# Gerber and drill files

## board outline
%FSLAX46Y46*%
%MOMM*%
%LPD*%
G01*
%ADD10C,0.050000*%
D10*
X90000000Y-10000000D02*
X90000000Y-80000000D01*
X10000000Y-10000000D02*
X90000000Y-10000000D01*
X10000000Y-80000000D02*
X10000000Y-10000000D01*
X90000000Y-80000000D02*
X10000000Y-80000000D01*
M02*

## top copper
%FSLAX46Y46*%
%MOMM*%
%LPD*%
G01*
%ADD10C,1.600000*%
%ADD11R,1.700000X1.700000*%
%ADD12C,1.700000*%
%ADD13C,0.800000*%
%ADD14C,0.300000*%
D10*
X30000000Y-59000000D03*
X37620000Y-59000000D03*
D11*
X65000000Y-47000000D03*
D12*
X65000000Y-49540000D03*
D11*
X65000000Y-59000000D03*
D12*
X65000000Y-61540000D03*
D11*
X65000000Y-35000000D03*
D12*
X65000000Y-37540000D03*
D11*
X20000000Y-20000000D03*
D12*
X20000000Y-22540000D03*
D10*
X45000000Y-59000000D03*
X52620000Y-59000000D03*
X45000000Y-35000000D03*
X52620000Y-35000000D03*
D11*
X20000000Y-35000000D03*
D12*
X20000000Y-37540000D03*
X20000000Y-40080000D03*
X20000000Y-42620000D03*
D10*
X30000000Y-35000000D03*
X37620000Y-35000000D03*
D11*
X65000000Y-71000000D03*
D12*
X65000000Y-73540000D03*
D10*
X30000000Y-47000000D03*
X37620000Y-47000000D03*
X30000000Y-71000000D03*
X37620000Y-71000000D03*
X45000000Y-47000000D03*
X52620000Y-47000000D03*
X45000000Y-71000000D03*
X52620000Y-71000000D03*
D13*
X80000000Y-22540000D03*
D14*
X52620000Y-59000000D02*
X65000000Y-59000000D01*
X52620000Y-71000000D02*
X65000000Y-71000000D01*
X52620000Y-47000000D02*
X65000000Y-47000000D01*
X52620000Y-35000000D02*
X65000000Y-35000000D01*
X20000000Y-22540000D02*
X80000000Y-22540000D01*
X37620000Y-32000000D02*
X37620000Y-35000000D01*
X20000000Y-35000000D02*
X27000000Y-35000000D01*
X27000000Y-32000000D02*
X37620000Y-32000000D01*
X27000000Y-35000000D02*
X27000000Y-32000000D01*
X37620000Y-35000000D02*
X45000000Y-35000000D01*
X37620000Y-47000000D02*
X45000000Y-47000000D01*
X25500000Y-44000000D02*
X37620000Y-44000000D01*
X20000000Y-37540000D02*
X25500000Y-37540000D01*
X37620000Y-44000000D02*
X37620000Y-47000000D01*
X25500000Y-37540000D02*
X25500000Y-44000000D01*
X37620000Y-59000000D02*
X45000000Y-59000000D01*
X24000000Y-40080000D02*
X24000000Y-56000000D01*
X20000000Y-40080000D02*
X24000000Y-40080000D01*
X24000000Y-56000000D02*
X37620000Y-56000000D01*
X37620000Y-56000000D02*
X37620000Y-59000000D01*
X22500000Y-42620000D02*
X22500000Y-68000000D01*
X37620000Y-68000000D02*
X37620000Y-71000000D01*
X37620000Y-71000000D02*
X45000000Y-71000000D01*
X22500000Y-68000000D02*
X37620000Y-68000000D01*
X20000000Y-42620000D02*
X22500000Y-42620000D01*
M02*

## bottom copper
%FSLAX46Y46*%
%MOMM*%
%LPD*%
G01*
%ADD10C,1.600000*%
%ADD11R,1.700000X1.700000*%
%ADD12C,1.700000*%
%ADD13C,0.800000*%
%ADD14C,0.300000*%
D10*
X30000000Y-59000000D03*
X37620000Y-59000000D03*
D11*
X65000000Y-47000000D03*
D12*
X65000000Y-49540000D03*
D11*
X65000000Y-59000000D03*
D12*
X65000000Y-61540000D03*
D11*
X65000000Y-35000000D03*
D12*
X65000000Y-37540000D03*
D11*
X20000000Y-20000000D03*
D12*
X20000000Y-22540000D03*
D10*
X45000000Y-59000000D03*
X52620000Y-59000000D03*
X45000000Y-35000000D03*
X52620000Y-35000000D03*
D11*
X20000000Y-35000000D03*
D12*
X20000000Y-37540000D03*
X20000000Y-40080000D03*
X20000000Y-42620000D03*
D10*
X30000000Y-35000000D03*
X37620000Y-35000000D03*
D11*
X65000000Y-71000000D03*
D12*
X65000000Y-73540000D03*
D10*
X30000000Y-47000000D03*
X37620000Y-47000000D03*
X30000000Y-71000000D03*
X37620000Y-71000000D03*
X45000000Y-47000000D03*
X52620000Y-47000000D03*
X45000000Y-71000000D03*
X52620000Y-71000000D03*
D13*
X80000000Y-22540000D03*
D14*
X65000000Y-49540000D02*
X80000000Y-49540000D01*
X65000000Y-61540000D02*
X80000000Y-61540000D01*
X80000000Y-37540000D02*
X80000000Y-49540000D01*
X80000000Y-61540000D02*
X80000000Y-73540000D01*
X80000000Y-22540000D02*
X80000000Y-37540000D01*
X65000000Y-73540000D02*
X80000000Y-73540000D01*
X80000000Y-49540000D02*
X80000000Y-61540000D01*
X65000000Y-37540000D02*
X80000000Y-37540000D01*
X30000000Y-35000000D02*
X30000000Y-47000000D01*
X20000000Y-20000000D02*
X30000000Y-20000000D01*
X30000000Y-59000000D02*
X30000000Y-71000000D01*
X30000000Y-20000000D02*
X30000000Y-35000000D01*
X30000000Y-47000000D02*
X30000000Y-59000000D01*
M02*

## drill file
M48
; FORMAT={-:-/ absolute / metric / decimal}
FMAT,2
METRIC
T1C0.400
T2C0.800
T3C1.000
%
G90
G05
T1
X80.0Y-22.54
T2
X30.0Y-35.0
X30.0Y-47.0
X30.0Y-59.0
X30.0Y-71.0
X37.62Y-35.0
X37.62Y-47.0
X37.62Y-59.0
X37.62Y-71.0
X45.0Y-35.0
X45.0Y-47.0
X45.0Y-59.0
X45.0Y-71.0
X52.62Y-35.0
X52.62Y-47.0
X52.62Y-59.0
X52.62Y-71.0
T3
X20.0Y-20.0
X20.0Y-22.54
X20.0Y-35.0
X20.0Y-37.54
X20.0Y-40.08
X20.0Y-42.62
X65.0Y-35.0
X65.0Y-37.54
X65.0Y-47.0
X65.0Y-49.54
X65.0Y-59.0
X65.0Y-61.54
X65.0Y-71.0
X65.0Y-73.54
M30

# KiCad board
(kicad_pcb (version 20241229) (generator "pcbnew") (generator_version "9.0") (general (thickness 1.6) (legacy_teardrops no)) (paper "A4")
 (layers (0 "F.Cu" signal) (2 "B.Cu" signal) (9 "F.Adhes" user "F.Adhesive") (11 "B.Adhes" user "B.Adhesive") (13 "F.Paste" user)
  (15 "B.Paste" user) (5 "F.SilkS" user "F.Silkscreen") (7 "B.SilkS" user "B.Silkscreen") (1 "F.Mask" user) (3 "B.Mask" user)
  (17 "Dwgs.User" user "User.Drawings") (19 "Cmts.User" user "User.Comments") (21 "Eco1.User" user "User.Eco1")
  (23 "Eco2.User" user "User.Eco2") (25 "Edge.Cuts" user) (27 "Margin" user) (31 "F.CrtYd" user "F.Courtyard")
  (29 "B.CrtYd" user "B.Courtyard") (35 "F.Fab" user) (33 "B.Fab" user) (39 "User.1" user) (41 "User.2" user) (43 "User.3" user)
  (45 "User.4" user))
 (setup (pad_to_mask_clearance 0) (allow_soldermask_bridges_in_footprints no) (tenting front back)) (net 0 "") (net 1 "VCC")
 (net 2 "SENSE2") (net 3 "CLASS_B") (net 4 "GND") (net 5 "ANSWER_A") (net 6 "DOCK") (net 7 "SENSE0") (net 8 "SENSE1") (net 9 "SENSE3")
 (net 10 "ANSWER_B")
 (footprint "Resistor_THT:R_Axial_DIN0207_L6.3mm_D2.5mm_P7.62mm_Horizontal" (layer "F.Cu") (at 30 59)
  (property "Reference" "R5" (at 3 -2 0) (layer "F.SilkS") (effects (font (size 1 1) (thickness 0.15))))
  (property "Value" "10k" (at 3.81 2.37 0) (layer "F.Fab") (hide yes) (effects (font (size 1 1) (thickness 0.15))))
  (pad "1" thru_hole circle (at 0 0) (size 1.6 1.6) (drill 0.8) (layers "*.Cu" "*.Mask") (remove_unused_layers no) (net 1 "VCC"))
  (pad "2" thru_hole circle (at 7.62 0) (size 1.6 1.6) (drill 0.8) (layers "*.Cu" "*.Mask") (remove_unused_layers no) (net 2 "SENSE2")))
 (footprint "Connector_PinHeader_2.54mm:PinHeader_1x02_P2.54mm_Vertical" (layer "F.Cu") (at 65 47)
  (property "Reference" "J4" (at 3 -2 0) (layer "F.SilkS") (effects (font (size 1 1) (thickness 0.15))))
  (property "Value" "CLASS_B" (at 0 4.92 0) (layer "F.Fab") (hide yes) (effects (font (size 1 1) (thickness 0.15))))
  (pad "1" thru_hole rect (at 0 0) (size 1.7 1.7) (drill 1) (layers "*.Cu" "*.Mask") (remove_unused_layers no) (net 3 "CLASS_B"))
  (pad "2" thru_hole circle (at 0 2.54) (size 1.7 1.7) (drill 1) (layers "*.Cu" "*.Mask") (remove_unused_layers no) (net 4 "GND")))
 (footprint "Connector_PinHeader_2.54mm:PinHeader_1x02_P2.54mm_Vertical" (layer "F.Cu") (at 65 59)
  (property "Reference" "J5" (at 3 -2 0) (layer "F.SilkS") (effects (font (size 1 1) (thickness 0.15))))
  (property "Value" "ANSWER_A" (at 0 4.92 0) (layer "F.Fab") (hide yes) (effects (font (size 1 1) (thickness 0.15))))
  (pad "1" thru_hole rect (at 0 0) (size 1.7 1.7) (drill 1) (layers "*.Cu" "*.Mask") (remove_unused_layers no) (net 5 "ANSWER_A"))
  (pad "2" thru_hole circle (at 0 2.54) (size 1.7 1.7) (drill 1) (layers "*.Cu" "*.Mask") (remove_unused_layers no) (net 4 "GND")))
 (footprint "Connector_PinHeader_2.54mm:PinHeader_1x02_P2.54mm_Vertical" (layer "F.Cu") (at 65 35)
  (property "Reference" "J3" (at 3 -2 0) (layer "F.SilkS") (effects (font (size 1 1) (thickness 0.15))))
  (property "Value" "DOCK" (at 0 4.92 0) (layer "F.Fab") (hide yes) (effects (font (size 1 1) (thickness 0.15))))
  (pad "1" thru_hole rect (at 0 0) (size 1.7 1.7) (drill 1) (layers "*.Cu" "*.Mask") (remove_unused_layers no) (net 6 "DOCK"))
  (pad "2" thru_hole circle (at 0 2.54) (size 1.7 1.7) (drill 1) (layers "*.Cu" "*.Mask") (remove_unused_layers no) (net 4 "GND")))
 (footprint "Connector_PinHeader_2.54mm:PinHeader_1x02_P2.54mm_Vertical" (layer "F.Cu") (at 20 20)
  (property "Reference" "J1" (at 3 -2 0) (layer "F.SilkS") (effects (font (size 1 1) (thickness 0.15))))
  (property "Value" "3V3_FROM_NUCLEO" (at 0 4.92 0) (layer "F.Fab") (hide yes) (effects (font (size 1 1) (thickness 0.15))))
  (pad "1" thru_hole rect (at 0 0) (size 1.7 1.7) (drill 1) (layers "*.Cu" "*.Mask") (remove_unused_layers no) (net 1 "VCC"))
  (pad "2" thru_hole circle (at 0 2.54) (size 1.7 1.7) (drill 1) (layers "*.Cu" "*.Mask") (remove_unused_layers no) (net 4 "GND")))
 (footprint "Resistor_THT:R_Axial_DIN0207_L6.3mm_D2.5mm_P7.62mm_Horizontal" (layer "F.Cu") (at 45 59)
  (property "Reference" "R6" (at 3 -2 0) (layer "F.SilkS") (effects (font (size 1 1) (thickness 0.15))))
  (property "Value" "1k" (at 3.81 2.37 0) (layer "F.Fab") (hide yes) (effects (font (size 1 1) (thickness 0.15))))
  (pad "1" thru_hole circle (at 0 0) (size 1.6 1.6) (drill 0.8) (layers "*.Cu" "*.Mask") (remove_unused_layers no) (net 2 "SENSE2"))
  (pad "2" thru_hole circle (at 7.62 0) (size 1.6 1.6) (drill 0.8) (layers "*.Cu" "*.Mask") (remove_unused_layers no) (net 5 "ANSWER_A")))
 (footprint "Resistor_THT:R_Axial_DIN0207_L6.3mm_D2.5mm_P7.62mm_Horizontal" (layer "F.Cu") (at 45 35)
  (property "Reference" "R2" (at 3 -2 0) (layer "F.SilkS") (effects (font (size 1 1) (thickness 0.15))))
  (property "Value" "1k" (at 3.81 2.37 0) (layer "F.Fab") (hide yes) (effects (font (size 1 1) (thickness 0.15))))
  (pad "1" thru_hole circle (at 0 0) (size 1.6 1.6) (drill 0.8) (layers "*.Cu" "*.Mask") (remove_unused_layers no) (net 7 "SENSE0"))
  (pad "2" thru_hole circle (at 7.62 0) (size 1.6 1.6) (drill 0.8) (layers "*.Cu" "*.Mask") (remove_unused_layers no) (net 6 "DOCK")))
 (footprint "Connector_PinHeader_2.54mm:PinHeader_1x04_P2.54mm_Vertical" (layer "F.Cu") (at 20 35)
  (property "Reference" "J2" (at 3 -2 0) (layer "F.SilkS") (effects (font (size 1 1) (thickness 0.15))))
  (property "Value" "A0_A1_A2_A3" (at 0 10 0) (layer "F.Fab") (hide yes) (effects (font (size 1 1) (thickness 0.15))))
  (pad "1" thru_hole rect (at 0 0) (size 1.7 1.7) (drill 1) (layers "*.Cu" "*.Mask") (remove_unused_layers no) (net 7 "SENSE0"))
  (pad "2" thru_hole circle (at 0 2.54) (size 1.7 1.7) (drill 1) (layers "*.Cu" "*.Mask") (remove_unused_layers no) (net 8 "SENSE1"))
  (pad "3" thru_hole circle (at 0 5.08) (size 1.7 1.7) (drill 1) (layers "*.Cu" "*.Mask") (remove_unused_layers no) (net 2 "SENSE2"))
  (pad "4" thru_hole circle (at 0 7.62) (size 1.7 1.7) (drill 1) (layers "*.Cu" "*.Mask") (remove_unused_layers no) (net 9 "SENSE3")))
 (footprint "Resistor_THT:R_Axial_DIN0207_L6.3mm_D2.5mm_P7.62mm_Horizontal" (layer "F.Cu") (at 30 35)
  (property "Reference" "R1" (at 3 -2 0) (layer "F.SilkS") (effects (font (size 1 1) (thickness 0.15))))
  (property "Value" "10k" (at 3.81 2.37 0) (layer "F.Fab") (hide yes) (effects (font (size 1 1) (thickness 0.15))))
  (pad "1" thru_hole circle (at 0 0) (size 1.6 1.6) (drill 0.8) (layers "*.Cu" "*.Mask") (remove_unused_layers no) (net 1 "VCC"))
  (pad "2" thru_hole circle (at 7.62 0) (size 1.6 1.6) (drill 0.8) (layers "*.Cu" "*.Mask") (remove_unused_layers no) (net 7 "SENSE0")))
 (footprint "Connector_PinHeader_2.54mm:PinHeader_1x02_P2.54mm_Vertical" (layer "F.Cu") (at 65 71)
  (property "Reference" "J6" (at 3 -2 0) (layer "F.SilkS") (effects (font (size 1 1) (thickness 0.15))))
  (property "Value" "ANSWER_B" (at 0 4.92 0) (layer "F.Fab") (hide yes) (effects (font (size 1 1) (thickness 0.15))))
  (pad "1" thru_hole rect (at 0 0) (size 1.7 1.7) (drill 1) (layers "*.Cu" "*.Mask") (remove_unused_layers no) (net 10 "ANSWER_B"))
  (pad "2" thru_hole circle (at 0 2.54) (size 1.7 1.7) (drill 1) (layers "*.Cu" "*.Mask") (remove_unused_layers no) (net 4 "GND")))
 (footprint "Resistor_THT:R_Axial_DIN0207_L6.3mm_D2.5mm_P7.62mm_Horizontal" (layer "F.Cu") (at 30 47)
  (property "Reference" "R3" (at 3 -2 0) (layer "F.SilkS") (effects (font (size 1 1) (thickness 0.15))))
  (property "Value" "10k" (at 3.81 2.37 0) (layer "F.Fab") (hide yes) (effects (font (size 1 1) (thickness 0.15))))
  (pad "1" thru_hole circle (at 0 0) (size 1.6 1.6) (drill 0.8) (layers "*.Cu" "*.Mask") (remove_unused_layers no) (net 1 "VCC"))
  (pad "2" thru_hole circle (at 7.62 0) (size 1.6 1.6) (drill 0.8) (layers "*.Cu" "*.Mask") (remove_unused_layers no) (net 8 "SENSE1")))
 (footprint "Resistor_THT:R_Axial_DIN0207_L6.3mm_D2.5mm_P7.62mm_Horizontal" (layer "F.Cu") (at 30 71)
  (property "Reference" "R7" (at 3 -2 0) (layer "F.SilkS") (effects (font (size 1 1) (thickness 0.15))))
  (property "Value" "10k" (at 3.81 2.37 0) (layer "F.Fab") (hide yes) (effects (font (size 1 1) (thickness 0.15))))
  (pad "1" thru_hole circle (at 0 0) (size 1.6 1.6) (drill 0.8) (layers "*.Cu" "*.Mask") (remove_unused_layers no) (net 1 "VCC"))
  (pad "2" thru_hole circle (at 7.62 0) (size 1.6 1.6) (drill 0.8) (layers "*.Cu" "*.Mask") (remove_unused_layers no) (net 9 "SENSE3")))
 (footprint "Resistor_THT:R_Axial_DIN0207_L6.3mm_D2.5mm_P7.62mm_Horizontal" (layer "F.Cu") (at 45 47)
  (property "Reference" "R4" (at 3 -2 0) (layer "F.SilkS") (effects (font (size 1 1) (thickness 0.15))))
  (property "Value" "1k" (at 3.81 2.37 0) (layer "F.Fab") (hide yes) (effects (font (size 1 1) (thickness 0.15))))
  (pad "1" thru_hole circle (at 0 0) (size 1.6 1.6) (drill 0.8) (layers "*.Cu" "*.Mask") (remove_unused_layers no) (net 8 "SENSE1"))
  (pad "2" thru_hole circle (at 7.62 0) (size 1.6 1.6) (drill 0.8) (layers "*.Cu" "*.Mask") (remove_unused_layers no) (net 3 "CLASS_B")))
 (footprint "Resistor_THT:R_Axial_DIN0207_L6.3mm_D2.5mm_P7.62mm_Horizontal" (layer "F.Cu") (at 45 71)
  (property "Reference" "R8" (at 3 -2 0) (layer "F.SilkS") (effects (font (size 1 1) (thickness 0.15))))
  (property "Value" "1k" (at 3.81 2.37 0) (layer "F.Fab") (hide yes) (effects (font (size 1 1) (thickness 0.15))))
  (pad "1" thru_hole circle (at 0 0) (size 1.6 1.6) (drill 0.8) (layers "*.Cu" "*.Mask") (remove_unused_layers no) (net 9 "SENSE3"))
  (pad "2" thru_hole circle (at 7.62 0) (size 1.6 1.6) (drill 0.8) (layers "*.Cu" "*.Mask") (remove_unused_layers no) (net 10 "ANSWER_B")))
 (gr_line (start 90 10) (end 90 80) (stroke (width 0.05) (type default)) (layer "Edge.Cuts"))
 (gr_line (start 10 10) (end 90 10) (stroke (width 0.05) (type default)) (layer "Edge.Cuts"))
 (gr_line (start 10 80) (end 10 10) (stroke (width 0.05) (type default)) (layer "Edge.Cuts"))
 (gr_line (start 90 80) (end 10 80) (stroke (width 0.05) (type default)) (layer "Edge.Cuts"))
 (segment (start 52.62 59) (end 65 59) (width 0.3) (layer "F.Cu") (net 5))
 (segment (start 52.62 71) (end 65 71) (width 0.3) (layer "F.Cu") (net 10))
 (segment (start 52.62 47) (end 65 47) (width 0.3) (layer "F.Cu") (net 3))
 (segment (start 52.62 35) (end 65 35) (width 0.3) (layer "F.Cu") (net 6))
 (segment (start 20 22.54) (end 80 22.54) (width 0.3) (layer "F.Cu") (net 4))
 (via (at 80 22.54) (size 0.8) (drill 0.4) (layers "F.Cu" "B.Cu") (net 4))
 (segment (start 65 49.54) (end 80 49.54) (width 0.3) (layer "B.Cu") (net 4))
 (segment (start 65 61.54) (end 80 61.54) (width 0.3) (layer "B.Cu") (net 4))
 (segment (start 80 37.54) (end 80 49.54) (width 0.3) (layer "B.Cu") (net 4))
 (segment (start 80 61.54) (end 80 73.54) (width 0.3) (layer "B.Cu") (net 4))
 (segment (start 80 22.54) (end 80 37.54) (width 0.3) (layer "B.Cu") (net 4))
 (segment (start 65 73.54) (end 80 73.54) (width 0.3) (layer "B.Cu") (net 4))
 (segment (start 80 49.54) (end 80 61.54) (width 0.3) (layer "B.Cu") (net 4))
 (segment (start 65 37.54) (end 80 37.54) (width 0.3) (layer "B.Cu") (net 4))
 (segment (start 37.62 32) (end 37.62 35) (width 0.3) (layer "F.Cu") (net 7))
 (segment (start 20 35) (end 27 35) (width 0.3) (layer "F.Cu") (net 7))
 (segment (start 27 32) (end 37.62 32) (width 0.3) (layer "F.Cu") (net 7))
 (segment (start 27 35) (end 27 32) (width 0.3) (layer "F.Cu") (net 7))
 (segment (start 37.62 35) (end 45 35) (width 0.3) (layer "F.Cu") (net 7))
 (segment (start 37.62 47) (end 45 47) (width 0.3) (layer "F.Cu") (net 8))
 (segment (start 25.5 44) (end 37.62 44) (width 0.3) (layer "F.Cu") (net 8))
 (segment (start 20 37.54) (end 25.5 37.54) (width 0.3) (layer "F.Cu") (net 8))
 (segment (start 37.62 44) (end 37.62 47) (width 0.3) (layer "F.Cu") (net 8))
 (segment (start 25.5 37.54) (end 25.5 44) (width 0.3) (layer "F.Cu") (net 8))
 (segment (start 37.62 59) (end 45 59) (width 0.3) (layer "F.Cu") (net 2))
 (segment (start 24 40.08) (end 24 56) (width 0.3) (layer "F.Cu") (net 2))
 (segment (start 20 40.08) (end 24 40.08) (width 0.3) (layer "F.Cu") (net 2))
 (segment (start 24 56) (end 37.62 56) (width 0.3) (layer "F.Cu") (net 2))
 (segment (start 37.62 56) (end 37.62 59) (width 0.3) (layer "F.Cu") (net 2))
 (segment (start 22.5 42.62) (end 22.5 68) (width 0.3) (layer "F.Cu") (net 9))
 (segment (start 37.62 68) (end 37.62 71) (width 0.3) (layer "F.Cu") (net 9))
 (segment (start 37.62 71) (end 45 71) (width 0.3) (layer "F.Cu") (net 9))
 (segment (start 22.5 68) (end 37.62 68) (width 0.3) (layer "F.Cu") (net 9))
 (segment (start 20 42.62) (end 22.5 42.62) (width 0.3) (layer "F.Cu") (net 9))
 (segment (start 30 35) (end 30 47) (width 0.3) (layer "B.Cu") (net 1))
 (segment (start 20 20) (end 30 20) (width 0.3) (layer "B.Cu") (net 1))
 (segment (start 30 59) (end 30 71) (width 0.3) (layer "B.Cu") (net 1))
 (segment (start 30 20) (end 30 35) (width 0.3) (layer "B.Cu") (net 1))
 (segment (start 30 47) (end 30 59) (width 0.3) (layer "B.Cu") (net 1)))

